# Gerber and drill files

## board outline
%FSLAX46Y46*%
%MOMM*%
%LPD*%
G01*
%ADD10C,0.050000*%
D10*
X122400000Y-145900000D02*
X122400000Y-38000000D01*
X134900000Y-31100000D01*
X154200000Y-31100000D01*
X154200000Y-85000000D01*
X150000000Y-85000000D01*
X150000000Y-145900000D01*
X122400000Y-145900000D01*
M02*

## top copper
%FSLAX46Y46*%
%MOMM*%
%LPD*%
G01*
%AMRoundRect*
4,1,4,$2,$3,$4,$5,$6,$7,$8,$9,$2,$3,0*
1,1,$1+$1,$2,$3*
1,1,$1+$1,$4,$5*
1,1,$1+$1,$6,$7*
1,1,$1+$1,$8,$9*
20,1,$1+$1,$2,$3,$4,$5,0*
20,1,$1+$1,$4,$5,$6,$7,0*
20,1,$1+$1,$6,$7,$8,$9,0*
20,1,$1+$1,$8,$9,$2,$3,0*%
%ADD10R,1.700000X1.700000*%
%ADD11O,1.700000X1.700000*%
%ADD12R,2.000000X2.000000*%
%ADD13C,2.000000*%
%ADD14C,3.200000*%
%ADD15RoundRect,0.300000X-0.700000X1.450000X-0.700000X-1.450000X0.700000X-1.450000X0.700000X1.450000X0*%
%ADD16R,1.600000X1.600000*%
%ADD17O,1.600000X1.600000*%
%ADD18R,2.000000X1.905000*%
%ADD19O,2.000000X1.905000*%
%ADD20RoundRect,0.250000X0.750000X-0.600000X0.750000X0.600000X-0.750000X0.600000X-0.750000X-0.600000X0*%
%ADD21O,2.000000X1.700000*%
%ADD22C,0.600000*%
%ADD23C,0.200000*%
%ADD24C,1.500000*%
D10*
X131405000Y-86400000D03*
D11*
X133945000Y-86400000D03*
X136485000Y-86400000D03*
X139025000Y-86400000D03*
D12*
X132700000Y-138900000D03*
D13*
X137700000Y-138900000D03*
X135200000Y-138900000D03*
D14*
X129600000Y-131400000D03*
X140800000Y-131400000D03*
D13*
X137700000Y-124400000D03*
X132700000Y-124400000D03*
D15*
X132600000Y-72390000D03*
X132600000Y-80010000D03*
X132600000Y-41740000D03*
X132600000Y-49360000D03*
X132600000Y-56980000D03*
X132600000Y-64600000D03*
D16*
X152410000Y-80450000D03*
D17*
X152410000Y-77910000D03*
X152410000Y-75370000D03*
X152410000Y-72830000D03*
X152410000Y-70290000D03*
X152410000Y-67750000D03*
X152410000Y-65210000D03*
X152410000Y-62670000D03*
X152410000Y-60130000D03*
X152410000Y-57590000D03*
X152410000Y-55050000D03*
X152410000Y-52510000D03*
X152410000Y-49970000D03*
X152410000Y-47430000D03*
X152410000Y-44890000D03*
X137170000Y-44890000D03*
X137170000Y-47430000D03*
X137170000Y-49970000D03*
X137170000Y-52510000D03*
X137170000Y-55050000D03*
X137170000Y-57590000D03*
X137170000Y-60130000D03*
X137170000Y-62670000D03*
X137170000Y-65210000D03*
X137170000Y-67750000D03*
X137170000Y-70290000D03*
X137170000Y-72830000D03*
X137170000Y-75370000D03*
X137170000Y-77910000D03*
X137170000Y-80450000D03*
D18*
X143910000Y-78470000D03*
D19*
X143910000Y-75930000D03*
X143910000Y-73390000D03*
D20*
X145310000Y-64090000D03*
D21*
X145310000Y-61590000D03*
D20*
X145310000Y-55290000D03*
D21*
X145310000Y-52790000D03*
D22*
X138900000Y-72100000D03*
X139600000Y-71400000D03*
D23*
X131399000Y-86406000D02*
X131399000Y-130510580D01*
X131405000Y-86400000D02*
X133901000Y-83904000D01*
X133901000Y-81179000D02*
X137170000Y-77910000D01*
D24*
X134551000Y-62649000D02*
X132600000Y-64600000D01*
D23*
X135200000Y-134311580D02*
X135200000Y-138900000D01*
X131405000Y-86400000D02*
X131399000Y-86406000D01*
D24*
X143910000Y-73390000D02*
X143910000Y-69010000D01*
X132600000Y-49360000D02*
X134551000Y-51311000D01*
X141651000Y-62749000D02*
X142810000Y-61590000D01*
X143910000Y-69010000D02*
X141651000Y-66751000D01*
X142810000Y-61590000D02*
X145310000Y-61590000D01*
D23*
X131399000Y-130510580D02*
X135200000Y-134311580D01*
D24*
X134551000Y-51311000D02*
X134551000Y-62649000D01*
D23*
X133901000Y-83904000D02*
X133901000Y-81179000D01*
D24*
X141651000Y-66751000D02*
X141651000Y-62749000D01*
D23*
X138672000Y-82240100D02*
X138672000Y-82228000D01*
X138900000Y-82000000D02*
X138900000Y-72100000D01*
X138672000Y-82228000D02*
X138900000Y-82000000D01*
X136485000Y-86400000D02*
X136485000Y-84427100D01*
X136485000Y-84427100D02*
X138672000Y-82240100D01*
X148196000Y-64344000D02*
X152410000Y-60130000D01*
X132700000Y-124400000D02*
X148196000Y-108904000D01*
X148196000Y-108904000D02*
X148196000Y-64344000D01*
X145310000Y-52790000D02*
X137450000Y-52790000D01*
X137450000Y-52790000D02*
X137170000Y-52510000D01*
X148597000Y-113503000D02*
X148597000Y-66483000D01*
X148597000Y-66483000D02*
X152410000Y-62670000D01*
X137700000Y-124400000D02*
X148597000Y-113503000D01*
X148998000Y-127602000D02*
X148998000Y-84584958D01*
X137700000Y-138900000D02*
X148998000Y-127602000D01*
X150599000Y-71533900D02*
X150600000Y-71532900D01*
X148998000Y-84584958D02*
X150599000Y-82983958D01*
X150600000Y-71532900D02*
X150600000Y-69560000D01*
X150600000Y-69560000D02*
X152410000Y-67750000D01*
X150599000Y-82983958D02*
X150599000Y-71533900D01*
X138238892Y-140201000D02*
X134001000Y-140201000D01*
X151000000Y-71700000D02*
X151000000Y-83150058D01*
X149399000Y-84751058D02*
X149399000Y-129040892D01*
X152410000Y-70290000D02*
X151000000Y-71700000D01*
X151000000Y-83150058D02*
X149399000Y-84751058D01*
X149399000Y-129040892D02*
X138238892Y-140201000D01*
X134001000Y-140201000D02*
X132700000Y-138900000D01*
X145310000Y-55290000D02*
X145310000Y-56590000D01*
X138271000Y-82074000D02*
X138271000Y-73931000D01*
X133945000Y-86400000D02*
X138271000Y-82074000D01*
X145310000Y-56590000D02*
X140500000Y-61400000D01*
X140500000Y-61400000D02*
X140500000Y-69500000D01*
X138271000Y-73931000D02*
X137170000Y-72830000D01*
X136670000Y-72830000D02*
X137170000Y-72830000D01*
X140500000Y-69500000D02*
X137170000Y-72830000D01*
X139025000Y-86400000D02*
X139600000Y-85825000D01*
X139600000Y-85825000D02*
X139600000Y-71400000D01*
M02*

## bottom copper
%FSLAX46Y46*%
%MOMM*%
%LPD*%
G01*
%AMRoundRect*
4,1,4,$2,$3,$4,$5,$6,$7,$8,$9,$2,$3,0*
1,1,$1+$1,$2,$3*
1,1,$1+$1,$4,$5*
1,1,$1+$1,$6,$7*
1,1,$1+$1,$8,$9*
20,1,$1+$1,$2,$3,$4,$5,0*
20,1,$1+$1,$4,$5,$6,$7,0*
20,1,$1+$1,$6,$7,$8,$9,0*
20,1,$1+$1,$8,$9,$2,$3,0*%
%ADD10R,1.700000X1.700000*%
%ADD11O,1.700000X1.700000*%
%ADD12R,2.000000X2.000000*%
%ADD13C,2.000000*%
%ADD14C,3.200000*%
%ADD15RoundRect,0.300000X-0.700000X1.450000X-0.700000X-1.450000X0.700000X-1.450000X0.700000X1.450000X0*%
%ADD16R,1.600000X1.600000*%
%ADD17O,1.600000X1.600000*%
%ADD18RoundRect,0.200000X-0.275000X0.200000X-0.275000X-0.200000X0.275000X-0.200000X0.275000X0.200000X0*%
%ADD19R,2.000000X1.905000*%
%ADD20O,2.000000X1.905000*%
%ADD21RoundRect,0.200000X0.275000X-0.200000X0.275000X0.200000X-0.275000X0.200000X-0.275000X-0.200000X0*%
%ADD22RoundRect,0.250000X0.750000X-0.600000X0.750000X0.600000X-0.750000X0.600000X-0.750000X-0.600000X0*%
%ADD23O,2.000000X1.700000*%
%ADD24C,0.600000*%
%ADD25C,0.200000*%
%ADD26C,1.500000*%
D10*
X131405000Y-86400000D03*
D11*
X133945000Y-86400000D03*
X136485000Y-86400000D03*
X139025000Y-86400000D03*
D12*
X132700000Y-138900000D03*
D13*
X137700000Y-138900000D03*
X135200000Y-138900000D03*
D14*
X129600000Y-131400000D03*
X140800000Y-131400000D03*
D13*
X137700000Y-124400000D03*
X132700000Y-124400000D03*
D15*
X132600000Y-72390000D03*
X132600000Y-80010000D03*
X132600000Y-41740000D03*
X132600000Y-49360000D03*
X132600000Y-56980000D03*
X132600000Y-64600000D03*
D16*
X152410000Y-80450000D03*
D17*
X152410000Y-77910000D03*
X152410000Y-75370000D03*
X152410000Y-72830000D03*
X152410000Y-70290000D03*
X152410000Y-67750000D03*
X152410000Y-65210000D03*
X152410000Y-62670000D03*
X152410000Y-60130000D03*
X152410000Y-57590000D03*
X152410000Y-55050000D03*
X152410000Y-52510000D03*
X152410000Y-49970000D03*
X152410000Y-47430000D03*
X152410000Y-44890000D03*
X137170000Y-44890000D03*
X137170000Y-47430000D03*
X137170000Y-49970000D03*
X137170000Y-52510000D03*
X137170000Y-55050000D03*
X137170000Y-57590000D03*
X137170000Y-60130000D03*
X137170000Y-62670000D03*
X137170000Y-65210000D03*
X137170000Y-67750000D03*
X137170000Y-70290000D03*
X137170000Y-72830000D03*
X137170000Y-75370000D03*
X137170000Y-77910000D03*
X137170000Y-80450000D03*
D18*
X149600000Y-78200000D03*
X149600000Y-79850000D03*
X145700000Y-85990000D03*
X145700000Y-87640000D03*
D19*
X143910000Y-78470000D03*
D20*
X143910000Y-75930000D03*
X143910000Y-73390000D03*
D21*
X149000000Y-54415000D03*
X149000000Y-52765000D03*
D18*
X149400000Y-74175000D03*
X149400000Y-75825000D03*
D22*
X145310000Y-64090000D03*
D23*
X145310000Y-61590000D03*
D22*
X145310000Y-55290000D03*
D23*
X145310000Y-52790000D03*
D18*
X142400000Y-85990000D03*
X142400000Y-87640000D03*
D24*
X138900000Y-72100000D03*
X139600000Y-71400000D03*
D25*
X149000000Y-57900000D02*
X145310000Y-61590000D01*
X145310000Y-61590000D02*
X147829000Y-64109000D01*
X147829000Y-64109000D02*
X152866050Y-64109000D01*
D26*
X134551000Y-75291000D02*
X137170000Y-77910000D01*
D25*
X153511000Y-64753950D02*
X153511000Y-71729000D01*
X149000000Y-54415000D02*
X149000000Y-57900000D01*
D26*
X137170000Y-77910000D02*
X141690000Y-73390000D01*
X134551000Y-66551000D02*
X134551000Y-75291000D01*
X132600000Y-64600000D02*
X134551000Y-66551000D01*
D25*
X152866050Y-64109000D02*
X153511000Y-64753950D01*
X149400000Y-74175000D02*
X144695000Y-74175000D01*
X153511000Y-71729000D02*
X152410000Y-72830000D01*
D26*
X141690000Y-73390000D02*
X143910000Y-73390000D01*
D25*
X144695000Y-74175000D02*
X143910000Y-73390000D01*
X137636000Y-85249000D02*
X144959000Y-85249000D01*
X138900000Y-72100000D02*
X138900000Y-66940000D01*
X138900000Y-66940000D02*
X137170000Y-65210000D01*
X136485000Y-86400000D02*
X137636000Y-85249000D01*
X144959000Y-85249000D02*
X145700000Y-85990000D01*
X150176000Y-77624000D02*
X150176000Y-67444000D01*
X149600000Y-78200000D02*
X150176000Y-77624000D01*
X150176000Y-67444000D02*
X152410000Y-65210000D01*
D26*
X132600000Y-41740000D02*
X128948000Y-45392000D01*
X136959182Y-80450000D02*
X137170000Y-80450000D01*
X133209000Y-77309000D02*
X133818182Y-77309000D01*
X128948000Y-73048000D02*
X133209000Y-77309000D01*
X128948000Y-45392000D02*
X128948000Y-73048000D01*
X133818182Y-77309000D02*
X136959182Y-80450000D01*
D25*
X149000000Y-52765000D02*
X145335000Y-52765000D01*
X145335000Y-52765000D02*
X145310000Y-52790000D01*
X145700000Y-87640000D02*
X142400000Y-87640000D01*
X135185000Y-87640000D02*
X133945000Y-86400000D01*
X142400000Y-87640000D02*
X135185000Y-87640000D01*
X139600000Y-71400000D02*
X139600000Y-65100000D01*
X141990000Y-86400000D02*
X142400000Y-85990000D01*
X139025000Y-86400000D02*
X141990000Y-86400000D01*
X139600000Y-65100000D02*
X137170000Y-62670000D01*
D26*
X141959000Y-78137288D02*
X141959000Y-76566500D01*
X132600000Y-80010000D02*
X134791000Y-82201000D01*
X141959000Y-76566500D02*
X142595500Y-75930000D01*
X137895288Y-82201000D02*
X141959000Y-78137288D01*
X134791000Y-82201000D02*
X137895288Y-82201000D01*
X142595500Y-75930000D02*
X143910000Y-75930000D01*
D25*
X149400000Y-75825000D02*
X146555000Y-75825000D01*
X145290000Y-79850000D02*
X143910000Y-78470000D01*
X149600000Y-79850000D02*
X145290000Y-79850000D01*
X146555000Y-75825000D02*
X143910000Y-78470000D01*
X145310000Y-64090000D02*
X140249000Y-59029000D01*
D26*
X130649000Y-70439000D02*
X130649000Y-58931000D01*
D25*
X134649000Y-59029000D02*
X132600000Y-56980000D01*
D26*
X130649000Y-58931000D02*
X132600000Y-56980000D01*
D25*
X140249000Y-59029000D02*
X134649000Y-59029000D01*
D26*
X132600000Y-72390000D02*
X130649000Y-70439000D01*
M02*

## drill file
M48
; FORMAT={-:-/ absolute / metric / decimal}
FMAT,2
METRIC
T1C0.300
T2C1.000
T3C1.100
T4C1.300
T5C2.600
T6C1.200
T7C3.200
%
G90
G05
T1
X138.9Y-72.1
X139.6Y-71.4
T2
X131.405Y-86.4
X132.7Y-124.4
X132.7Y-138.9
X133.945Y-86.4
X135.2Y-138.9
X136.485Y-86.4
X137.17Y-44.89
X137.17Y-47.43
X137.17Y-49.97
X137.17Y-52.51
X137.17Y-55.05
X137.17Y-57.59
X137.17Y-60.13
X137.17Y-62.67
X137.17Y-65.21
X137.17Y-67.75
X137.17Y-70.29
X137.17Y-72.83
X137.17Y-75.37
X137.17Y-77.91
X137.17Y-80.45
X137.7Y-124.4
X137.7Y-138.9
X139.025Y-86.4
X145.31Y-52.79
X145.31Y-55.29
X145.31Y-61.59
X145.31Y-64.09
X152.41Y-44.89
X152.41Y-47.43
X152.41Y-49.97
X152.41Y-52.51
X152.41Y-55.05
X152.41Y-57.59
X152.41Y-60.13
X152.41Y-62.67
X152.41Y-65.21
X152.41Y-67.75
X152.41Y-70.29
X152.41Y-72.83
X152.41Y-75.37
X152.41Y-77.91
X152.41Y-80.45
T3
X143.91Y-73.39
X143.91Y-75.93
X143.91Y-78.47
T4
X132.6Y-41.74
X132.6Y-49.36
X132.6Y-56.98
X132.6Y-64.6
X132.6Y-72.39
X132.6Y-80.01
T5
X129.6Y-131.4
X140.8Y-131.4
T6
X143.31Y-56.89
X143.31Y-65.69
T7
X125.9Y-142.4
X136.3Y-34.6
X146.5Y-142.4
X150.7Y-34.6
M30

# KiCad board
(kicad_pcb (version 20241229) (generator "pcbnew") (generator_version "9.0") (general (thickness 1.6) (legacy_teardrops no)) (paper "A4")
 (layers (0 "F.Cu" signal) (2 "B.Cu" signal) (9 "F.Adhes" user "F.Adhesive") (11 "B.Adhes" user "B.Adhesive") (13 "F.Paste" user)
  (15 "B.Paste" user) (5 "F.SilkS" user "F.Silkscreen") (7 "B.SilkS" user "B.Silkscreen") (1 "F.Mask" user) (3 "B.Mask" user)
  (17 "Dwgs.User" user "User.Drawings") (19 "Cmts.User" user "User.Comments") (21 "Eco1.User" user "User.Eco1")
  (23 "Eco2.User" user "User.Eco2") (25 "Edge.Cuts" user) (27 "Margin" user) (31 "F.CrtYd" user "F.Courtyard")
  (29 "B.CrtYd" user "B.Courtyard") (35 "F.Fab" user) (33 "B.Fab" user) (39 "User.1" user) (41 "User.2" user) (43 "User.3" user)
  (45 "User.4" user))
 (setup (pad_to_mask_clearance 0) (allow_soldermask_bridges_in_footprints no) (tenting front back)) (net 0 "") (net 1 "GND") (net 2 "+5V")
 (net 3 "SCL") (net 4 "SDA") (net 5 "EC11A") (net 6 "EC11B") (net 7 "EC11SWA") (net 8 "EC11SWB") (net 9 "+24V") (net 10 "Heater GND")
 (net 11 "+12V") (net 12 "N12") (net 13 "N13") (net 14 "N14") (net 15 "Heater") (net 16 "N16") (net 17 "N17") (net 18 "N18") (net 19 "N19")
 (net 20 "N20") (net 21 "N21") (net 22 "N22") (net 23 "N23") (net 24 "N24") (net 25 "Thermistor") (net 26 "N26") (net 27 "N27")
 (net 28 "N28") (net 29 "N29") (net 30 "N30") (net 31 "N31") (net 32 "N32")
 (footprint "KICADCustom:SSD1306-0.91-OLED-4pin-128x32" (layer "F.Cu") (at 129.215 122.9 90)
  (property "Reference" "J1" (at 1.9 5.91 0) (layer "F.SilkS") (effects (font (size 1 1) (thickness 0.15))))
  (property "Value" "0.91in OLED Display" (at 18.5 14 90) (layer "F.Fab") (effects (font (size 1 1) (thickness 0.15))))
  (pad "1" thru_hole rect (at 36.5 2.19 90) (size 1.7 1.7) (drill 1) (layers "*.Cu" "*.Mask") (remove_unused_layers no) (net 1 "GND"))
  (pad "2" thru_hole oval (at 36.5 4.73 90) (size 1.7 1.7) (drill 1) (layers "*.Cu" "*.Mask") (remove_unused_layers no) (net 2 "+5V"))
  (pad "3" thru_hole oval (at 36.5 7.27 90) (size 1.7 1.7) (drill 1) (layers "*.Cu" "*.Mask") (remove_unused_layers no) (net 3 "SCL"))
  (pad "4" thru_hole oval (at 36.5 9.81 90) (size 1.7 1.7) (drill 1) (layers "*.Cu" "*.Mask") (remove_unused_layers no) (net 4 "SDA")))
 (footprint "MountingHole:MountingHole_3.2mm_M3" (layer "F.Cu") (at 146.5 142.4)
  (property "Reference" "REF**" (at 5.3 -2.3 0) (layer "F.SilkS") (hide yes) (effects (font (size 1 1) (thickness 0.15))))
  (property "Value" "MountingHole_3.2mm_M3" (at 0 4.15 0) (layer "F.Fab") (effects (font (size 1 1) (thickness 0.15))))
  (pad "" np_thru_hole circle (at 0 0) (size 3.2 3.2) (drill 3.2) (layers "*.Cu" "*.Mask")))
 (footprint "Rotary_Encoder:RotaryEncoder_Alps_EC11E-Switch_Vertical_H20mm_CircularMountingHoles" (layer "F.Cu") (at 132.7 138.9 90)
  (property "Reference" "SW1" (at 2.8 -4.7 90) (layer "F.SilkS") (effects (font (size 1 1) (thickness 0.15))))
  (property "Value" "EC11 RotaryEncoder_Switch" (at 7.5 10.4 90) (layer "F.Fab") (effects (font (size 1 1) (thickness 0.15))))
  (pad "A" thru_hole rect (at 0 0 90) (size 2 2) (drill 1) (layers "*.Cu" "*.Mask") (remove_unused_layers no) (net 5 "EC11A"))
  (pad "B" thru_hole circle (at 0 5 90) (size 2 2) (drill 1) (layers "*.Cu" "*.Mask") (remove_unused_layers no) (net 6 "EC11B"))
  (pad "C" thru_hole circle (at 0 2.5 90) (size 2 2) (drill 1) (layers "*.Cu" "*.Mask") (remove_unused_layers no) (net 1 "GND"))
  (pad "MP" thru_hole circle (at 7.5 -3.1 90) (size 3.2 3.2) (drill 2.6) (layers "*.Cu" "*.Mask") (remove_unused_layers no))
  (pad "MP" thru_hole circle (at 7.5 8.1 90) (size 3.2 3.2) (drill 2.6) (layers "*.Cu" "*.Mask") (remove_unused_layers no))
  (pad "S1" thru_hole circle (at 14.5 5 90) (size 2 2) (drill 1) (layers "*.Cu" "*.Mask") (remove_unused_layers no) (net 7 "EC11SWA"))
  (pad "S2" thru_hole circle (at 14.5 0 90) (size 2 2) (drill 1) (layers "*.Cu" "*.Mask") (remove_unused_layers no) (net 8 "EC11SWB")))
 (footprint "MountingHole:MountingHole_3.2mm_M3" (layer "F.Cu") (at 136.3 34.6)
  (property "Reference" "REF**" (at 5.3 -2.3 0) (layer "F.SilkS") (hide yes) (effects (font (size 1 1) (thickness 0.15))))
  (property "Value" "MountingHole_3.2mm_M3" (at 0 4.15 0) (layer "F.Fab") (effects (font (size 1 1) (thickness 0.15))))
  (pad "" np_thru_hole circle (at 0 0) (size 3.2 3.2) (drill 3.2) (layers "*.Cu" "*.Mask")))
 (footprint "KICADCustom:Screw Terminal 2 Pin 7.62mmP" (layer "F.Cu") (at 132.6 72.39 -90)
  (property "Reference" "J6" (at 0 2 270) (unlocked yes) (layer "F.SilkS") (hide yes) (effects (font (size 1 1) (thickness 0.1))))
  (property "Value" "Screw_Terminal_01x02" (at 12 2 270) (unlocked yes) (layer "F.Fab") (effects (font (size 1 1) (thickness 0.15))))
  (pad "1" thru_hole roundrect (at 0 0 270) (size 3.5 2) (drill 1.3) (layers "*.Cu" "*.Mask") (remove_unused_layers no)
   (roundrect_rratio 0.15) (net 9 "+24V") (thermal_bridge_angle 45))
  (pad "2" thru_hole roundrect (at 7.62 0 270) (size 3.5 2) (drill 1.3) (layers "*.Cu" "*.Mask") (remove_unused_layers no)
   (roundrect_rratio 0.15) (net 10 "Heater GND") (thermal_bridge_angle 45)))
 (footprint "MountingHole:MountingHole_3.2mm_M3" (layer "F.Cu") (at 150.7 34.6)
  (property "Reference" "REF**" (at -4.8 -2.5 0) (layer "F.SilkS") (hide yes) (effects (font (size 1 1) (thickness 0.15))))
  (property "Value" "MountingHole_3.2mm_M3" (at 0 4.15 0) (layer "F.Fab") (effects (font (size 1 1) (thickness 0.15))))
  (pad "" np_thru_hole circle (at 0 0) (size 3.2 3.2) (drill 3.2) (layers "*.Cu" "*.Mask")))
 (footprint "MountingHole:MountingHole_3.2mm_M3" (layer "F.Cu") (at 125.9 142.4)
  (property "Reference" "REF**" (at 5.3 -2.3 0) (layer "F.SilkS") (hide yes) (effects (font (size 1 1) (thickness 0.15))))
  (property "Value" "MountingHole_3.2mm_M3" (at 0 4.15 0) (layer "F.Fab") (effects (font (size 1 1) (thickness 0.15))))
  (pad "" np_thru_hole circle (at 0 0) (size 3.2 3.2) (drill 3.2) (layers "*.Cu" "*.Mask")))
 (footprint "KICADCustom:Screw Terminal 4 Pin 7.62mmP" (layer "F.Cu") (at 132.6 41.74 -90)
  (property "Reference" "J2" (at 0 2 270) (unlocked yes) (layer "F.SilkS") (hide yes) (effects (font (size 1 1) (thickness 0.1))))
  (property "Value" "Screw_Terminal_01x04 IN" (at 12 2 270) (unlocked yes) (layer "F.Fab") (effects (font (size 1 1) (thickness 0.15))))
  (pad "1" thru_hole roundrect (at 0 0 270) (size 3.5 2) (drill 1.3) (layers "*.Cu" "*.Mask") (remove_unused_layers no)
   (roundrect_rratio 0.15) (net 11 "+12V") (thermal_bridge_angle 45))
  (pad "2" thru_hole roundrect (at 7.62 0 270) (size 3.5 2) (drill 1.3) (layers "*.Cu" "*.Mask") (remove_unused_layers no)
   (roundrect_rratio 0.15) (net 1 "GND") (thermal_bridge_angle 45))
  (pad "3" thru_hole roundrect (at 15.24 0 270) (size 3.5 2) (drill 1.3) (layers "*.Cu" "*.Mask") (remove_unused_layers no)
   (roundrect_rratio 0.15) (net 9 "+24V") (thermal_bridge_angle 45))
  (pad "4" thru_hole roundrect (at 22.86 0 270) (size 3.5 2) (drill 1.3) (layers "*.Cu" "*.Mask") (remove_unused_layers no)
   (roundrect_rratio 0.15) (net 1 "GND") (thermal_bridge_angle 45)))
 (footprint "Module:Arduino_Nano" (layer "F.Cu") (at 152.41 80.45 180)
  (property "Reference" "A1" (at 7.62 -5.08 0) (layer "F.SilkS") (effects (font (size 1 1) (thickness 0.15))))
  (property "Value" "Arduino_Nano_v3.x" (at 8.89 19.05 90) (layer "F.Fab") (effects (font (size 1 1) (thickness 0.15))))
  (pad "1" thru_hole rect (at 0 0 180) (size 1.6 1.6) (drill 1) (layers "*.Cu" "*.Mask") (remove_unused_layers no) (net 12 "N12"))
  (pad "2" thru_hole oval (at 0 2.54 180) (size 1.6 1.6) (drill 1) (layers "*.Cu" "*.Mask") (remove_unused_layers no) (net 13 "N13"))
  (pad "3" thru_hole oval (at 0 5.08 180) (size 1.6 1.6) (drill 1) (layers "*.Cu" "*.Mask") (remove_unused_layers no) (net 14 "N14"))
  (pad "4" thru_hole oval (at 0 7.62 180) (size 1.6 1.6) (drill 1) (layers "*.Cu" "*.Mask") (remove_unused_layers no) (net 1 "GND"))
  (pad "5" thru_hole oval (at 0 10.16 180) (size 1.6 1.6) (drill 1) (layers "*.Cu" "*.Mask") (remove_unused_layers no) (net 5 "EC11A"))
  (pad "6" thru_hole oval (at 0 12.7 180) (size 1.6 1.6) (drill 1) (layers "*.Cu" "*.Mask") (remove_unused_layers no) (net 6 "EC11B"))
  (pad "7" thru_hole oval (at 0 15.24 180) (size 1.6 1.6) (drill 1) (layers "*.Cu" "*.Mask") (remove_unused_layers no) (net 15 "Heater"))
  (pad "8" thru_hole oval (at 0 17.78 180) (size 1.6 1.6) (drill 1) (layers "*.Cu" "*.Mask") (remove_unused_layers no) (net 7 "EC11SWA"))
  (pad "9" thru_hole oval (at 0 20.32 180) (size 1.6 1.6) (drill 1) (layers "*.Cu" "*.Mask") (remove_unused_layers no) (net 8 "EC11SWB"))
  (pad "10" thru_hole oval (at 0 22.86 180) (size 1.6 1.6) (drill 1) (layers "*.Cu" "*.Mask") (remove_unused_layers no) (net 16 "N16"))
  (pad "11" thru_hole oval (at 0 25.4 180) (size 1.6 1.6) (drill 1) (layers "*.Cu" "*.Mask") (remove_unused_layers no) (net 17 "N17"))
  (pad "12" thru_hole oval (at 0 27.94 180) (size 1.6 1.6) (drill 1) (layers "*.Cu" "*.Mask") (remove_unused_layers no) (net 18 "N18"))
  (pad "13" thru_hole oval (at 0 30.48 180) (size 1.6 1.6) (drill 1) (layers "*.Cu" "*.Mask") (remove_unused_layers no) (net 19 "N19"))
  (pad "14" thru_hole oval (at 0 33.02 180) (size 1.6 1.6) (drill 1) (layers "*.Cu" "*.Mask") (remove_unused_layers no) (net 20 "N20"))
  (pad "15" thru_hole oval (at 0 35.56 180) (size 1.6 1.6) (drill 1) (layers "*.Cu" "*.Mask") (remove_unused_layers no) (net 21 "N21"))
  (pad "16" thru_hole oval (at 15.24 35.56 180) (size 1.6 1.6) (drill 1) (layers "*.Cu" "*.Mask") (remove_unused_layers no) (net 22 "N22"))
  (pad "17" thru_hole oval (at 15.24 33.02 180) (size 1.6 1.6) (drill 1) (layers "*.Cu" "*.Mask") (remove_unused_layers no) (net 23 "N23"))
  (pad "18" thru_hole oval (at 15.24 30.48 180) (size 1.6 1.6) (drill 1) (layers "*.Cu" "*.Mask") (remove_unused_layers no) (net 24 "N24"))
  (pad "19" thru_hole oval (at 15.24 27.94 180) (size 1.6 1.6) (drill 1) (layers "*.Cu" "*.Mask") (remove_unused_layers no)
   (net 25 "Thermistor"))
  (pad "20" thru_hole oval (at 15.24 25.4 180) (size 1.6 1.6) (drill 1) (layers "*.Cu" "*.Mask") (remove_unused_layers no) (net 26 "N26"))
  (pad "21" thru_hole oval (at 15.24 22.86 180) (size 1.6 1.6) (drill 1) (layers "*.Cu" "*.Mask") (remove_unused_layers no) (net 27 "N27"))
  (pad "22" thru_hole oval (at 15.24 20.32 180) (size 1.6 1.6) (drill 1) (layers "*.Cu" "*.Mask") (remove_unused_layers no) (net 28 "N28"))
  (pad "23" thru_hole oval (at 15.24 17.78 180) (size 1.6 1.6) (drill 1) (layers "*.Cu" "*.Mask") (remove_unused_layers no) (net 4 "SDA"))
  (pad "24" thru_hole oval (at 15.24 15.24 180) (size 1.6 1.6) (drill 1) (layers "*.Cu" "*.Mask") (remove_unused_layers no) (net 3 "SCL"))
  (pad "25" thru_hole oval (at 15.24 12.7 180) (size 1.6 1.6) (drill 1) (layers "*.Cu" "*.Mask") (remove_unused_layers no) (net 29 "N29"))
  (pad "26" thru_hole oval (at 15.24 10.16 180) (size 1.6 1.6) (drill 1) (layers "*.Cu" "*.Mask") (remove_unused_layers no) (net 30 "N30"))
  (pad "27" thru_hole oval (at 15.24 7.62 180) (size 1.6 1.6) (drill 1) (layers "*.Cu" "*.Mask") (remove_unused_layers no) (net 2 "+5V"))
  (pad "28" thru_hole oval (at 15.24 5.08 180) (size 1.6 1.6) (drill 1) (layers "*.Cu" "*.Mask") (remove_unused_layers no) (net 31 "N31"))
  (pad "29" thru_hole oval (at 15.24 2.54 180) (size 1.6 1.6) (drill 1) (layers "*.Cu" "*.Mask") (remove_unused_layers no) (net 1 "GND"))
  (pad "30" thru_hole oval (at 15.24 0 180) (size 1.6 1.6) (drill 1) (layers "*.Cu" "*.Mask") (remove_unused_layers no) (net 11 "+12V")))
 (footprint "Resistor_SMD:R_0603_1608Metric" (layer "B.Cu") (at 149.6 79.025 -90)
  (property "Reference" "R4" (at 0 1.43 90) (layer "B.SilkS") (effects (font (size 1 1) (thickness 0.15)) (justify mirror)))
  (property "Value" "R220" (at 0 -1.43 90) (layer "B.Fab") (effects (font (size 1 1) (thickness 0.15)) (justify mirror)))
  (pad "1" smd roundrect (at -0.825 0 270) (size 0.8 0.95) (layers "B.Cu" "B.Mask" "B.Paste") (roundrect_rratio 0.25) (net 15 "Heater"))
  (pad "2" smd roundrect (at 0.825 0 270) (size 0.8 0.95) (layers "B.Cu" "B.Mask" "B.Paste") (roundrect_rratio 0.25) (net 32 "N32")))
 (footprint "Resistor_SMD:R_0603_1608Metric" (layer "B.Cu") (at 145.7 86.815 -90)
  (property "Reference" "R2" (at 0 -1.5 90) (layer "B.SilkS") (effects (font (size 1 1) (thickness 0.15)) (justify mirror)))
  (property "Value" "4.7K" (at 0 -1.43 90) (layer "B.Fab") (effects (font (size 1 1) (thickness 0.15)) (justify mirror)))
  (pad "1" smd roundrect (at -0.825 0 270) (size 0.8 0.95) (layers "B.Cu" "B.Mask" "B.Paste") (roundrect_rratio 0.25) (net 3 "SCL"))
  (pad "2" smd roundrect (at 0.825 0 270) (size 0.8 0.95) (layers "B.Cu" "B.Mask" "B.Paste") (roundrect_rratio 0.25) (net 2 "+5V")))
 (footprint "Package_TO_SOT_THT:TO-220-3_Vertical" (layer "B.Cu") (at 143.91 78.47 90)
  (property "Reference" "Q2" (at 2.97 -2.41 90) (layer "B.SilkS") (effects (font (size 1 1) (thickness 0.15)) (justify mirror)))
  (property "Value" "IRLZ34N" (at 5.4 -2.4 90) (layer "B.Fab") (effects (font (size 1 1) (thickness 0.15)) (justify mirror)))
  (pad "1" thru_hole rect (at 0 0 90) (size 1.905 2) (drill 1.1) (layers "*.Cu" "*.Mask") (remove_unused_layers no) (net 32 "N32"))
  (pad "2" thru_hole oval (at 2.54 0 90) (size 1.905 2) (drill 1.1) (layers "*.Cu" "*.Mask") (remove_unused_layers no) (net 10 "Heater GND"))
  (pad "3" thru_hole oval (at 5.08 0 90) (size 1.905 2) (drill 1.1) (layers "*.Cu" "*.Mask") (remove_unused_layers no) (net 1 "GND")))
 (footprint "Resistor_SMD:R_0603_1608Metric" (layer "B.Cu") (at 149 53.59 90)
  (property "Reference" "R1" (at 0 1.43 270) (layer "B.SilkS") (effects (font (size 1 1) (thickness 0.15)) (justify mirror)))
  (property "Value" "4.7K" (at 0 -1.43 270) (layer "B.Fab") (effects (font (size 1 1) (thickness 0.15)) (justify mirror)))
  (pad "1" smd roundrect (at -0.825 0 90) (size 0.8 0.95) (layers "B.Cu" "B.Mask" "B.Paste") (roundrect_rratio 0.25) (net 1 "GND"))
  (pad "2" smd roundrect (at 0.825 0 90) (size 0.8 0.95) (layers "B.Cu" "B.Mask" "B.Paste") (roundrect_rratio 0.25) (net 25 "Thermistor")))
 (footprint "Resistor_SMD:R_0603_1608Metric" (layer "B.Cu") (at 149.4 75 -90)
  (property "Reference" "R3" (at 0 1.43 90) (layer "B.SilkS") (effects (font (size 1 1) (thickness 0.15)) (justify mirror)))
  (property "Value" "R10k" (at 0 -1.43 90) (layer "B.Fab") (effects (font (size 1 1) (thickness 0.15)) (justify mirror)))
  (pad "1" smd roundrect (at -0.825 0 270) (size 0.8 0.95) (layers "B.Cu" "B.Mask" "B.Paste") (roundrect_rratio 0.25) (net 1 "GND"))
  (pad "2" smd roundrect (at 0.825 0 270) (size 0.8 0.95) (layers "B.Cu" "B.Mask" "B.Paste") (roundrect_rratio 0.25) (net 32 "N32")))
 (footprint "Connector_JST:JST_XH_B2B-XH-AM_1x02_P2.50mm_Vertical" (layer "B.Cu") (at 145.31 64.09 90)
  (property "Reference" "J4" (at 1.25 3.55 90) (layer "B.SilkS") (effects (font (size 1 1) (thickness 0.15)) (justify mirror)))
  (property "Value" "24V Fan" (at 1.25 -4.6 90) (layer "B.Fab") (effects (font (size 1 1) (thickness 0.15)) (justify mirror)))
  (pad "" np_thru_hole circle (at -1.6 -2 90) (size 1.2 1.2) (drill 1.2) (layers "*.Cu" "*.Mask"))
  (pad "1" thru_hole roundrect (at 0 0 90) (size 1.7 2) (drill 1) (layers "*.Cu" "*.Mask") (remove_unused_layers no)
   (roundrect_rratio 0.147059) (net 9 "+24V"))
  (pad "2" thru_hole oval (at 2.5 0 90) (size 1.7 2) (drill 1) (layers "*.Cu" "*.Mask") (remove_unused_layers no) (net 1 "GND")))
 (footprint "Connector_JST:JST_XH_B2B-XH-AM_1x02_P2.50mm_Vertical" (layer "B.Cu") (at 145.31 55.29 90)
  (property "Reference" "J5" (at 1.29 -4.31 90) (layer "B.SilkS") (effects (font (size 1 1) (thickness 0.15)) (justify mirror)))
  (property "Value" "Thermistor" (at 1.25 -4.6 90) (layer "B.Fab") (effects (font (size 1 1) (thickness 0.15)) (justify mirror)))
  (pad "" np_thru_hole circle (at -1.6 -2 90) (size 1.2 1.2) (drill 1.2) (layers "*.Cu" "*.Mask"))
  (pad "1" thru_hole roundrect (at 0 0 90) (size 1.7 2) (drill 1) (layers "*.Cu" "*.Mask") (remove_unused_layers no)
   (roundrect_rratio 0.147059) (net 2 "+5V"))
  (pad "2" thru_hole oval (at 2.5 0 90) (size 1.7 2) (drill 1) (layers "*.Cu" "*.Mask") (remove_unused_layers no) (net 25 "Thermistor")))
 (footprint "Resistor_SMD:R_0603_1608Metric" (layer "B.Cu") (at 142.4 86.815 -90)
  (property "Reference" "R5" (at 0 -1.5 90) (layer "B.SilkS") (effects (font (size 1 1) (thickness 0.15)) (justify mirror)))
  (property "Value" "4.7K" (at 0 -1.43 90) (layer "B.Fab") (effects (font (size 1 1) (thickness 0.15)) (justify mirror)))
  (pad "1" smd roundrect (at -0.825 0 270) (size 0.8 0.95) (layers "B.Cu" "B.Mask" "B.Paste") (roundrect_rratio 0.25) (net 4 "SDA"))
  (pad "2" smd roundrect (at 0.825 0 270) (size 0.8 0.95) (layers "B.Cu" "B.Mask" "B.Paste") (roundrect_rratio 0.25) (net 2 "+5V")))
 (gr_poly
  (pts (xy 122.4 145.9) (xy 122.4 38) (xy 134.9 31.1) (xy 154.2 31.1) (xy 154.2 85) (xy 150 85) (xy 150 145.9))
  (stroke (width 0.05) (type solid)) (fill no) (layer "Edge.Cuts"))
 (segment (start 131.399 86.406) (end 131.399 130.51058) (width 0.2) (layer "F.Cu") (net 1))
 (segment (start 131.405 86.4) (end 133.901 83.904) (width 0.2) (layer "F.Cu") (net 1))
 (segment (start 133.901 81.179) (end 137.17 77.91) (width 0.2) (layer "F.Cu") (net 1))
 (segment (start 134.551 62.649) (end 132.6 64.6) (width 1.5) (layer "F.Cu") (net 1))
 (segment (start 135.2 134.31158) (end 135.2 138.9) (width 0.2) (layer "F.Cu") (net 1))
 (segment (start 131.405 86.4) (end 131.399 86.406) (width 0.2) (layer "F.Cu") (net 1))
 (segment (start 143.91 73.39) (end 143.91 69.01) (width 1.5) (layer "F.Cu") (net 1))
 (segment (start 132.6 49.36) (end 134.551 51.311) (width 1.5) (layer "F.Cu") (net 1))
 (segment (start 141.651 62.749) (end 142.81 61.59) (width 1.5) (layer "F.Cu") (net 1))
 (segment (start 143.91 69.01) (end 141.651 66.751) (width 1.5) (layer "F.Cu") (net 1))
 (segment (start 142.81 61.59) (end 145.31 61.59) (width 1.5) (layer "F.Cu") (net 1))
 (segment (start 131.399 130.51058) (end 135.2 134.31158) (width 0.2) (layer "F.Cu") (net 1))
 (segment (start 134.551 51.311) (end 134.551 62.649) (width 1.5) (layer "F.Cu") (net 1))
 (segment (start 133.901 83.904) (end 133.901 81.179) (width 0.2) (layer "F.Cu") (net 1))
 (segment (start 141.651 66.751) (end 141.651 62.749) (width 1.5) (layer "F.Cu") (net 1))
 (segment (start 149 57.9) (end 145.31 61.59) (width 0.2) (layer "B.Cu") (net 1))
 (segment (start 145.31 61.59) (end 147.829 64.109) (width 0.2) (layer "B.Cu") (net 1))
 (segment (start 147.829 64.109) (end 152.86605 64.109) (width 0.2) (layer "B.Cu") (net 1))
 (segment (start 134.551 75.291) (end 137.17 77.91) (width 1.5) (layer "B.Cu") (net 1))
 (segment (start 153.511 64.75395) (end 153.511 71.729) (width 0.2) (layer "B.Cu") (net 1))
 (segment (start 149 54.415) (end 149 57.9) (width 0.2) (layer "B.Cu") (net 1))
 (segment (start 137.17 77.91) (end 141.69 73.39) (width 1.5) (layer "B.Cu") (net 1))
 (segment (start 134.551 66.551) (end 134.551 75.291) (width 1.5) (layer "B.Cu") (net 1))
 (segment (start 132.6 64.6) (end 134.551 66.551) (width 1.5) (layer "B.Cu") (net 1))
 (segment (start 152.86605 64.109) (end 153.511 64.75395) (width 0.2) (layer "B.Cu") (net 1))
 (segment (start 149.4 74.175) (end 144.695 74.175) (width 0.2) (layer "B.Cu") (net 1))
 (segment (start 153.511 71.729) (end 152.41 72.83) (width 0.2) (layer "B.Cu") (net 1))
 (segment (start 141.69 73.39) (end 143.91 73.39) (width 1.5) (layer "B.Cu") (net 1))
 (segment (start 144.695 74.175) (end 143.91 73.39) (width 0.2) (layer "B.Cu") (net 1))
 (segment (start 138.672 82.2401) (end 138.672 82.228) (width 0.2) (layer "F.Cu") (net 3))
 (segment (start 138.9 82) (end 138.9 72.1) (width 0.2) (layer "F.Cu") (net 3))
 (segment (start 138.672 82.228) (end 138.9 82) (width 0.2) (layer "F.Cu") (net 3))
 (segment (start 136.485 86.4) (end 136.485 84.4271) (width 0.2) (layer "F.Cu") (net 3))
 (segment (start 136.485 84.4271) (end 138.672 82.2401) (width 0.2) (layer "F.Cu") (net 3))
 (via (at 138.9 72.1) (size 0.6) (drill 0.3) (layers "F.Cu" "B.Cu") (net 3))
 (segment (start 137.636 85.249) (end 144.959 85.249) (width 0.2) (layer "B.Cu") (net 3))
 (segment (start 138.9 72.1) (end 138.9 66.94) (width 0.2) (layer "B.Cu") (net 3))
 (segment (start 138.9 66.94) (end 137.17 65.21) (width 0.2) (layer "B.Cu") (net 3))
 (segment (start 136.485 86.4) (end 137.636 85.249) (width 0.2) (layer "B.Cu") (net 3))
 (segment (start 144.959 85.249) (end 145.7 85.99) (width 0.2) (layer "B.Cu") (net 3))
 (segment (start 150.176 77.624) (end 150.176 67.444) (width 0.2) (layer "B.Cu") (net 15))
 (segment (start 149.6 78.2) (end 150.176 77.624) (width 0.2) (layer "B.Cu") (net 15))
 (segment (start 150.176 67.444) (end 152.41 65.21) (width 0.2) (layer "B.Cu") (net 15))
 (segment (start 148.196 64.344) (end 152.41 60.13) (width 0.2) (layer "F.Cu") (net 8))
 (segment (start 132.7 124.4) (end 148.196 108.904) (width 0.2) (layer "F.Cu") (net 8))
 (segment (start 148.196 108.904) (end 148.196 64.344) (width 0.2) (layer "F.Cu") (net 8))
 (segment (start 132.6 41.74) (end 128.948 45.392) (width 1.5) (layer "B.Cu") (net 11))
 (segment (start 136.959182 80.45) (end 137.17 80.45) (width 1.5) (layer "B.Cu") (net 11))
 (segment (start 133.209 77.309) (end 133.818182 77.309) (width 1.5) (layer "B.Cu") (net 11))
 (segment (start 128.948 73.048) (end 133.209 77.309) (width 1.5) (layer "B.Cu") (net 11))
 (segment (start 128.948 45.392) (end 128.948 73.048) (width 1.5) (layer "B.Cu") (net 11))
 (segment (start 133.818182 77.309) (end 136.959182 80.45) (width 1.5) (layer "B.Cu") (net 11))
 (segment (start 145.31 52.79) (end 137.45 52.79) (width 0.2) (layer "F.Cu") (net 25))
 (segment (start 137.45 52.79) (end 137.17 52.51) (width 0.2) (layer "F.Cu") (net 25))
 (segment (start 149 52.765) (end 145.335 52.765) (width 0.2) (layer "B.Cu") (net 25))
 (segment (start 145.335 52.765) (end 145.31 52.79) (width 0.2) (layer "B.Cu") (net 25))
 (segment (start 148.597 113.503) (end 148.597 66.483) (width 0.2) (layer "F.Cu") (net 7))
 (segment (start 148.597 66.483) (end 152.41 62.67) (width 0.2) (layer "F.Cu") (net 7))
 (segment (start 137.7 124.4) (end 148.597 113.503) (width 0.2) (layer "F.Cu") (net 7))
 (segment (start 148.998 127.602) (end 148.998 84.584958) (width 0.2) (layer "F.Cu") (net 6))
 (segment (start 137.7 138.9) (end 148.998 127.602) (width 0.2) (layer "F.Cu") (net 6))
 (segment (start 150.599 71.5339) (end 150.6 71.5329) (width 0.2) (layer "F.Cu") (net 6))
 (segment (start 148.998 84.584958) (end 150.599 82.983958) (width 0.2) (layer "F.Cu") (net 6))
 (segment (start 150.6 71.5329) (end 150.6 69.56) (width 0.2) (layer "F.Cu") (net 6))
 (segment (start 150.6 69.56) (end 152.41 67.75) (width 0.2) (layer "F.Cu") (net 6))
 (segment (start 150.599 82.983958) (end 150.599 71.5339) (width 0.2) (layer "F.Cu") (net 6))
 (segment (start 138.238892 140.201) (end 134.001 140.201) (width 0.2) (layer "F.Cu") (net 5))
 (segment (start 151 71.7) (end 151 83.150058) (width 0.2) (layer "F.Cu") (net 5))
 (segment (start 149.399 84.751058) (end 149.399 129.040892) (width 0.2) (layer "F.Cu") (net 5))
 (segment (start 152.41 70.29) (end 151 71.7) (width 0.2) (layer "F.Cu") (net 5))
 (segment (start 151 83.150058) (end 149.399 84.751058) (width 0.2) (layer "F.Cu") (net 5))
 (segment (start 149.399 129.040892) (end 138.238892 140.201) (width 0.2) (layer "F.Cu") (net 5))
 (segment (start 134.001 140.201) (end 132.7 138.9) (width 0.2) (layer "F.Cu") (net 5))
 (segment (start 145.31 55.29) (end 145.31 56.59) (width 0.2) (layer "F.Cu") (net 2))
 (segment (start 138.271 82.074) (end 138.271 73.931) (width 0.2) (layer "F.Cu") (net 2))
 (segment (start 133.945 86.4) (end 138.271 82.074) (width 0.2) (layer "F.Cu") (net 2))
 (segment (start 145.31 56.59) (end 140.5 61.4) (width 0.2) (layer "F.Cu") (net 2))
 (segment (start 140.5 61.4) (end 140.5 69.5) (width 0.2) (layer "F.Cu") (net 2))
 (segment (start 138.271 73.931) (end 137.17 72.83) (width 0.2) (layer "F.Cu") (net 2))
 (segment (start 136.67 72.83) (end 137.17 72.83) (width 0.2) (layer "F.Cu") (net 2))
 (segment (start 140.5 69.5) (end 137.17 72.83) (width 0.2) (layer "F.Cu") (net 2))
 (segment (start 145.7 87.64) (end 142.4 87.64) (width 0.2) (layer "B.Cu") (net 2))
 (segment (start 135.185 87.64) (end 133.945 86.4) (width 0.2) (layer "B.Cu") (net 2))
 (segment (start 142.4 87.64) (end 135.185 87.64) (width 0.2) (layer "B.Cu") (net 2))
 (segment (start 139.025 86.4) (end 139.6 85.825) (width 0.2) (layer "F.Cu") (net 4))
 (segment (start 139.6 85.825) (end 139.6 71.4) (width 0.2) (layer "F.Cu") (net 4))
 (via (at 139.6 71.4) (size 0.6) (drill 0.3) (layers "F.Cu" "B.Cu") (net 4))
 (segment (start 139.6 71.4) (end 139.6 65.1) (width 0.2) (layer "B.Cu") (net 4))
 (segment (start 141.99 86.4) (end 142.4 85.99) (width 0.2) (layer "B.Cu") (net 4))
 (segment (start 139.025 86.4) (end 141.99 86.4) (width 0.2) (layer "B.Cu") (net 4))
 (segment (start 139.6 65.1) (end 137.17 62.67) (width 0.2) (layer "B.Cu") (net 4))
 (segment (start 141.959 78.137288) (end 141.959 76.5665) (width 1.5) (layer "B.Cu") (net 10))
 (segment (start 132.6 80.01) (end 134.791 82.201) (width 1.5) (layer "B.Cu") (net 10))
 (segment (start 141.959 76.5665) (end 142.5955 75.93) (width 1.5) (layer "B.Cu") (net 10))
 (segment (start 137.895288 82.201) (end 141.959 78.137288) (width 1.5) (layer "B.Cu") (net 10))
 (segment (start 134.791 82.201) (end 137.895288 82.201) (width 1.5) (layer "B.Cu") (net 10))
 (segment (start 142.5955 75.93) (end 143.91 75.93) (width 1.5) (layer "B.Cu") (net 10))
 (segment (start 149.4 75.825) (end 146.555 75.825) (width 0.2) (layer "B.Cu") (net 32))
 (segment (start 145.29 79.85) (end 143.91 78.47) (width 0.2) (layer "B.Cu") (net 32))
 (segment (start 149.6 79.85) (end 145.29 79.85) (width 0.2) (layer "B.Cu") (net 32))
 (segment (start 146.555 75.825) (end 143.91 78.47) (width 0.2) (layer "B.Cu") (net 32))
 (segment (start 145.31 64.09) (end 140.249 59.029) (width 0.2) (layer "B.Cu") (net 9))
 (segment (start 130.649 70.439) (end 130.649 58.931) (width 1.5) (layer "B.Cu") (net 9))
 (segment (start 134.649 59.029) (end 132.6 56.98) (width 0.2) (layer "B.Cu") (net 9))
 (segment (start 130.649 58.931) (end 132.6 56.98) (width 1.5) (layer "B.Cu") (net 9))
 (segment (start 140.249 59.029) (end 134.649 59.029) (width 0.2) (layer "B.Cu") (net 9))
 (segment (start 132.6 72.39) (end 130.649 70.439) (width 1.5) (layer "B.Cu") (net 9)))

